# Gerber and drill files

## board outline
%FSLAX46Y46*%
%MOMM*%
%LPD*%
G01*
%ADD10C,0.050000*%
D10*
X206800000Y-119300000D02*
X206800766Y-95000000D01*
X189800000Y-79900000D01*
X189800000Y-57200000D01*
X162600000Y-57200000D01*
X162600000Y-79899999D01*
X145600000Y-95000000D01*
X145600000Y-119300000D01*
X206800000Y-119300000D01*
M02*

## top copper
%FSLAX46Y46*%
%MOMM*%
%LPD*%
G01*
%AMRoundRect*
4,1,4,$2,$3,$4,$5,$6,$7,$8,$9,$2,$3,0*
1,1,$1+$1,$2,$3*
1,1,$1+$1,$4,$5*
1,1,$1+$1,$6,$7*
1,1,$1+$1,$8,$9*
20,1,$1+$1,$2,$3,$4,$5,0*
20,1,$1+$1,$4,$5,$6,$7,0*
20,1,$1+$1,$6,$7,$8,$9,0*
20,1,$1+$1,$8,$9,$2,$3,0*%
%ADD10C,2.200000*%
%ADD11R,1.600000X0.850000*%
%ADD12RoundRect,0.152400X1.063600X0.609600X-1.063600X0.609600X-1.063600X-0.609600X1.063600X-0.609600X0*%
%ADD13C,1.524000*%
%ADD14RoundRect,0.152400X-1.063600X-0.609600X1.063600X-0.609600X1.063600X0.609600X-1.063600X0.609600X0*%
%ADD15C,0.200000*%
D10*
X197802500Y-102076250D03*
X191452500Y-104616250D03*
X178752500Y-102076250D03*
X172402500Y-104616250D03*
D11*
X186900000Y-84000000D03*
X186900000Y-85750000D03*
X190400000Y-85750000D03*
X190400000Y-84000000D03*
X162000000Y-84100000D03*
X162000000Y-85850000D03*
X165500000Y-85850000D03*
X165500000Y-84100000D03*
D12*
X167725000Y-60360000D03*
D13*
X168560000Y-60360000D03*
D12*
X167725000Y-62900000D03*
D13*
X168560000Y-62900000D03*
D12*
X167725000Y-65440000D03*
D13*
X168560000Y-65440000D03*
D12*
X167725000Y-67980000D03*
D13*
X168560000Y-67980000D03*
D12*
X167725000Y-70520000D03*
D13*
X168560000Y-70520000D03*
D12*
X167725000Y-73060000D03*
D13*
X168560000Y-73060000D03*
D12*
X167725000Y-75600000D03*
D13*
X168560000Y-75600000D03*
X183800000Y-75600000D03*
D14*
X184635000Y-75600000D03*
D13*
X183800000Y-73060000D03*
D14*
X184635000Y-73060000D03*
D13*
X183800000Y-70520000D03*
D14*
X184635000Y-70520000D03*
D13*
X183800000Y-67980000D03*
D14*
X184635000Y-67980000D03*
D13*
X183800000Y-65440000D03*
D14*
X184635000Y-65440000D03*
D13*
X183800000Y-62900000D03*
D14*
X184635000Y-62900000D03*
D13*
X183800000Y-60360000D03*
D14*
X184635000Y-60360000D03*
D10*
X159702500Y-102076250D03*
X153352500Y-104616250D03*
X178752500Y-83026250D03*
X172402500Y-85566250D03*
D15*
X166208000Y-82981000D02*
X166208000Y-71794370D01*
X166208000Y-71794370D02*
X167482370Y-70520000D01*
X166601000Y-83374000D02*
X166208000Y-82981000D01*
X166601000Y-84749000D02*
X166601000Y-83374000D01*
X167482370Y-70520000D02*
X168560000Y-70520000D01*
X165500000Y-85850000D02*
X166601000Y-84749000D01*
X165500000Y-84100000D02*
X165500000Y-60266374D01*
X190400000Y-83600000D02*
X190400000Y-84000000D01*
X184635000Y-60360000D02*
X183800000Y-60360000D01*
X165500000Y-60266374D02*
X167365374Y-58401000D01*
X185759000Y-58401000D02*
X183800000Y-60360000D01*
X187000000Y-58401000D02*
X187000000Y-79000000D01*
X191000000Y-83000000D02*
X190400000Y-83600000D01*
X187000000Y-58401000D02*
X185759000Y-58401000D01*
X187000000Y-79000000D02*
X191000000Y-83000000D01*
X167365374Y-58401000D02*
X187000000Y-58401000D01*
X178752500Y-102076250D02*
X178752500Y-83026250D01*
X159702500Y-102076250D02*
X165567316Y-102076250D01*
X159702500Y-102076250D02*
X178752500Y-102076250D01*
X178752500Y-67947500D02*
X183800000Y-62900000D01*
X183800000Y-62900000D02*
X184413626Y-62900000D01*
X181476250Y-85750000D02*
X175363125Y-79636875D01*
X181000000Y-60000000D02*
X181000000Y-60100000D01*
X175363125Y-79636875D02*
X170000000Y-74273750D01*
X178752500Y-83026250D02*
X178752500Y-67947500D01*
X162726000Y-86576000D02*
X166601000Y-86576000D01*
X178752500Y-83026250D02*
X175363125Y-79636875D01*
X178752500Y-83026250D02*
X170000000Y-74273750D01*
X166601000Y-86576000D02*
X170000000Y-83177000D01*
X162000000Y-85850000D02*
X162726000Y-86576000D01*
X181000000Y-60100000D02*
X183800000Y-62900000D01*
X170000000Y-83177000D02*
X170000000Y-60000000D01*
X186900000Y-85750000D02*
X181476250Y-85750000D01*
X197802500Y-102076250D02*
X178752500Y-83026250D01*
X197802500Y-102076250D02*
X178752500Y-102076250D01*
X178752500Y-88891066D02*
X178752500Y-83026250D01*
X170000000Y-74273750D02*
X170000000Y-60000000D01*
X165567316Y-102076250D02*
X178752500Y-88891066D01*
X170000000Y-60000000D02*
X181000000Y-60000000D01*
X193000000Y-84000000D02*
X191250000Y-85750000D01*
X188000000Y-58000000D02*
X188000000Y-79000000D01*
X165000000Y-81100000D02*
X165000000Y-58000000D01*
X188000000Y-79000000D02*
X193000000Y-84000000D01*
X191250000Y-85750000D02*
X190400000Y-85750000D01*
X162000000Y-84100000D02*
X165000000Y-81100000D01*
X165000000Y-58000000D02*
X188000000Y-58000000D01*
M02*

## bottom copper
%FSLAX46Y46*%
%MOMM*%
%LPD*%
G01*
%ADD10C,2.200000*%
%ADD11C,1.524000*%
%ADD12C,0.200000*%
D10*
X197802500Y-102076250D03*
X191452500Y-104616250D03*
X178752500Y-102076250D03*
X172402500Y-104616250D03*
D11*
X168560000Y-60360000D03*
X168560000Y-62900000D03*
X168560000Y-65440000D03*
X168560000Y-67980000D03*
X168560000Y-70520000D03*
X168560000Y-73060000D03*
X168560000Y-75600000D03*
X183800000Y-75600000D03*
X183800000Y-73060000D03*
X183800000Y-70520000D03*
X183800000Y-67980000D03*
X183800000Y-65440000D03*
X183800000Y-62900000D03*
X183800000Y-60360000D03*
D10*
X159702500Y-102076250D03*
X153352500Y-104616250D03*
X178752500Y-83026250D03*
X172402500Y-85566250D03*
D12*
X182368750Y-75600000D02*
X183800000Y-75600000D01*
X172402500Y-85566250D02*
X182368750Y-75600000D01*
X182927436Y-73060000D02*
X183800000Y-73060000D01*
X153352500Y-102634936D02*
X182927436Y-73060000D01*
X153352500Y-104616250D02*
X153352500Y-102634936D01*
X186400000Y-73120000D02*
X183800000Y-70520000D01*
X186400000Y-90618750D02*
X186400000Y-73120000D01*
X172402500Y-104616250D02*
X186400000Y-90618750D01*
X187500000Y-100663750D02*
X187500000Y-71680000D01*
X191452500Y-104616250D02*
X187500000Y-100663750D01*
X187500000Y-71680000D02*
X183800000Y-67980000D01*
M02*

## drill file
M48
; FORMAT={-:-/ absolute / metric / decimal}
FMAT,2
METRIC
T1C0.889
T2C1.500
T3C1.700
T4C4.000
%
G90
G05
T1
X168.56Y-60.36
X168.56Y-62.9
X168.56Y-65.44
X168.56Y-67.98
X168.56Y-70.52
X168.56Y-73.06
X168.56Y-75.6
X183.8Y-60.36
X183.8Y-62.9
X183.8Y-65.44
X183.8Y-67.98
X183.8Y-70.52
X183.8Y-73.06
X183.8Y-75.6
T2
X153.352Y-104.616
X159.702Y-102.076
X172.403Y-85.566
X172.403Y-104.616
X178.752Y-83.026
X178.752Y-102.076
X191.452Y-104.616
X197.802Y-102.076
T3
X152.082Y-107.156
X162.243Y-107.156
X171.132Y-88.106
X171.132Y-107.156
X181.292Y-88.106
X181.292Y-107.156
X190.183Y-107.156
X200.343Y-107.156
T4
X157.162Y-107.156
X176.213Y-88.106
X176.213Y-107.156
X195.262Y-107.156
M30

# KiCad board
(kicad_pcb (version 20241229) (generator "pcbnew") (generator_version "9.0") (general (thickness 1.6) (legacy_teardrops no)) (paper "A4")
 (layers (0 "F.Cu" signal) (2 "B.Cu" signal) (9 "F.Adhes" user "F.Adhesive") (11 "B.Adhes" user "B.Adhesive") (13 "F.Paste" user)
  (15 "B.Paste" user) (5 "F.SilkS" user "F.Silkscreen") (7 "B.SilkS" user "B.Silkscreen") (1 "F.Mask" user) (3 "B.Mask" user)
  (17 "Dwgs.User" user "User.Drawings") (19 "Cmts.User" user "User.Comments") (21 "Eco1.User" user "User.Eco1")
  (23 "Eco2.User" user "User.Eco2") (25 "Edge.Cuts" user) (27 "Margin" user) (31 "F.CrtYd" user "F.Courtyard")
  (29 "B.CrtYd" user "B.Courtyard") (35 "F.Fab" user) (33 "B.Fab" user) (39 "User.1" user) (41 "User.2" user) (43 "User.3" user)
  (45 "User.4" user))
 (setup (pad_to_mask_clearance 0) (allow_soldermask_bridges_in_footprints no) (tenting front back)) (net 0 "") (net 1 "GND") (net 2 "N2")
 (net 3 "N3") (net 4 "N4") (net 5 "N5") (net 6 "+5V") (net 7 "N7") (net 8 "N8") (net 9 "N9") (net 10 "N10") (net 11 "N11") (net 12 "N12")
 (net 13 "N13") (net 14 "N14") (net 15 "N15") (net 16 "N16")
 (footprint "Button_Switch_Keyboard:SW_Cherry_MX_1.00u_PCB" (layer "F.Cu") (at 197.8025 102.07625)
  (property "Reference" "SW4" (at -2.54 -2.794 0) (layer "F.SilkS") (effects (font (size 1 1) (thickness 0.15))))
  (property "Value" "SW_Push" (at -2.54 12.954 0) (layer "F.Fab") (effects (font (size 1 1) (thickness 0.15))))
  (pad "" np_thru_hole circle (at -7.62 5.08) (size 1.7 1.7) (drill 1.7) (layers "*.Cu" "*.Mask"))
  (pad "" np_thru_hole circle (at -2.54 5.08) (size 4 4) (drill 4) (layers "*.Cu" "*.Mask"))
  (pad "" np_thru_hole circle (at 2.54 5.08) (size 1.7 1.7) (drill 1.7) (layers "*.Cu" "*.Mask"))
  (pad "1" thru_hole circle (at 0 0) (size 2.2 2.2) (drill 1.5) (layers "*.Cu" "*.Mask") (remove_unused_layers no) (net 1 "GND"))
  (pad "2" thru_hole circle (at -6.35 2.54) (size 2.2 2.2) (drill 1.5) (layers "*.Cu" "*.Mask") (remove_unused_layers no) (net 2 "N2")))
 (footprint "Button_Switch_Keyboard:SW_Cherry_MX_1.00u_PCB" (layer "F.Cu") (at 178.7525 102.07625)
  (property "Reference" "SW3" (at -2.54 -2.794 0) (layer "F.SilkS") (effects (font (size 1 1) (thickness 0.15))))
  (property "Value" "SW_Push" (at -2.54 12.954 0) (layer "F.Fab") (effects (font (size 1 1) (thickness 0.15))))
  (pad "" np_thru_hole circle (at -7.62 5.08) (size 1.7 1.7) (drill 1.7) (layers "*.Cu" "*.Mask"))
  (pad "" np_thru_hole circle (at -2.54 5.08) (size 4 4) (drill 4) (layers "*.Cu" "*.Mask"))
  (pad "" np_thru_hole circle (at 2.54 5.08) (size 1.7 1.7) (drill 1.7) (layers "*.Cu" "*.Mask"))
  (pad "1" thru_hole circle (at 0 0) (size 2.2 2.2) (drill 1.5) (layers "*.Cu" "*.Mask") (remove_unused_layers no) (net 1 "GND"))
  (pad "2" thru_hole circle (at -6.35 2.54) (size 2.2 2.2) (drill 1.5) (layers "*.Cu" "*.Mask") (remove_unused_layers no) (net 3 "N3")))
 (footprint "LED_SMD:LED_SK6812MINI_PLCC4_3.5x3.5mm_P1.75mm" (layer "F.Cu") (at 188.65 84.875)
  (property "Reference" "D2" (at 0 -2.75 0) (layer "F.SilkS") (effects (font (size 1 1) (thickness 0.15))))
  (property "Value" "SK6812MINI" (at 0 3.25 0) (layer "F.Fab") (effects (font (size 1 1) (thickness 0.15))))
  (pad "1" smd rect (at -1.75 -0.875) (size 1.6 0.85) (layers "F.Cu" "F.Mask" "F.Paste") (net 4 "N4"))
  (pad "2" smd rect (at -1.75 0.875) (size 1.6 0.85) (layers "F.Cu" "F.Mask" "F.Paste") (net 1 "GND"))
  (pad "3" smd rect (at 1.75 0.875) (size 1.6 0.85) (layers "F.Cu" "F.Mask" "F.Paste") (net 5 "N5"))
  (pad "4" smd rect (at 1.75 -0.875) (size 1.6 0.85) (layers "F.Cu" "F.Mask" "F.Paste") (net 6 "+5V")))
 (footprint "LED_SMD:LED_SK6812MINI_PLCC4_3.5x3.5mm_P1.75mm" (layer "F.Cu") (at 163.75 84.975)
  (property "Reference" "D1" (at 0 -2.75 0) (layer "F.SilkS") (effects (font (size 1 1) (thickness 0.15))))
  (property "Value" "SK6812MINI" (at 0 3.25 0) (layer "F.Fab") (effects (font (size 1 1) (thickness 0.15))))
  (pad "1" smd rect (at -1.75 -0.875) (size 1.6 0.85) (layers "F.Cu" "F.Mask" "F.Paste") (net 5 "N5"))
  (pad "2" smd rect (at -1.75 0.875) (size 1.6 0.85) (layers "F.Cu" "F.Mask" "F.Paste") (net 1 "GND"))
  (pad "3" smd rect (at 1.75 0.875) (size 1.6 0.85) (layers "F.Cu" "F.Mask" "F.Paste") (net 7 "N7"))
  (pad "4" smd rect (at 1.75 -0.875) (size 1.6 0.85) (layers "F.Cu" "F.Mask" "F.Paste") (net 6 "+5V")))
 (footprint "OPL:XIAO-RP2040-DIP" (layer "F.Cu") (at 176.18 67.98)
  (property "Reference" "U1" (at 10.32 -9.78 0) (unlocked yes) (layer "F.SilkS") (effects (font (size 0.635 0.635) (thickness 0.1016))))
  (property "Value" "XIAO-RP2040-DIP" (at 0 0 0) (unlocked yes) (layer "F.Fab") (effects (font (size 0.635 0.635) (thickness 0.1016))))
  (pad "1" smd roundrect (at -8.455 -7.62 180) (size 2.432 1.524) (layers "F.Cu" "F.Mask") (roundrect_rratio 0.1) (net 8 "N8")
   (thermal_bridge_angle 45))
  (pad "1" thru_hole circle (at -7.62 -7.62 180) (size 1.524 1.524) (drill 0.889) (layers "*.Cu" "*.Mask") (remove_unused_layers no)
   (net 8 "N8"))
  (pad "2" smd roundrect (at -8.455 -5.08 180) (size 2.432 1.524) (layers "F.Cu" "F.Mask") (roundrect_rratio 0.1) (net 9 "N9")
   (thermal_bridge_angle 45))
  (pad "2" thru_hole circle (at -7.62 -5.08 180) (size 1.524 1.524) (drill 0.889) (layers "*.Cu" "*.Mask") (remove_unused_layers no)
   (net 9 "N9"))
  (pad "3" smd roundrect (at -8.455 -2.54 180) (size 2.432 1.524) (layers "F.Cu" "F.Mask") (roundrect_rratio 0.1) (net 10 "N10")
   (thermal_bridge_angle 45))
  (pad "3" thru_hole circle (at -7.62 -2.54 180) (size 1.524 1.524) (drill 0.889) (layers "*.Cu" "*.Mask") (remove_unused_layers no)
   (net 10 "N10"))
  (pad "4" smd roundrect (at -8.455 0 180) (size 2.432 1.524) (layers "F.Cu" "F.Mask") (roundrect_rratio 0.1) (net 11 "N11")
   (thermal_bridge_angle 45))
  (pad "4" thru_hole circle (at -7.62 0 180) (size 1.524 1.524) (drill 0.889) (layers "*.Cu" "*.Mask") (remove_unused_layers no)
   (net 11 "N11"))
  (pad "5" smd roundrect (at -8.455 2.54 180) (size 2.432 1.524) (layers "F.Cu" "F.Mask") (roundrect_rratio 0.1) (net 7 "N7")
   (thermal_bridge_angle 45))
  (pad "5" thru_hole circle (at -7.62 2.54 180) (size 1.524 1.524) (drill 0.889) (layers "*.Cu" "*.Mask") (remove_unused_layers no)
   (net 7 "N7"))
  (pad "6" smd roundrect (at -8.455 5.08 180) (size 2.432 1.524) (layers "F.Cu" "F.Mask") (roundrect_rratio 0.1) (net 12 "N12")
   (thermal_bridge_angle 45))
  (pad "6" thru_hole circle (at -7.62 5.08 180) (size 1.524 1.524) (drill 0.889) (layers "*.Cu" "*.Mask") (remove_unused_layers no)
   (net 12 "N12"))
  (pad "7" smd roundrect (at -8.455 7.62 180) (size 2.432 1.524) (layers "F.Cu" "F.Mask") (roundrect_rratio 0.1) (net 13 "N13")
   (thermal_bridge_angle 45))
  (pad "7" thru_hole circle (at -7.62 7.62 180) (size 1.524 1.524) (drill 0.889) (layers "*.Cu" "*.Mask") (remove_unused_layers no)
   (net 13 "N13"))
  (pad "8" thru_hole circle (at 7.62 7.62) (size 1.524 1.524) (drill 0.889) (layers "*.Cu" "*.Mask") (remove_unused_layers no)
   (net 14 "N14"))
  (pad "8" smd roundrect (at 8.455 7.62) (size 2.432 1.524) (layers "F.Cu" "F.Mask") (roundrect_rratio 0.1) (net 14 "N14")
   (thermal_bridge_angle 45))
  (pad "9" thru_hole circle (at 7.62 5.08) (size 1.524 1.524) (drill 0.889) (layers "*.Cu" "*.Mask") (remove_unused_layers no)
   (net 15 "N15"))
  (pad "9" smd roundrect (at 8.455 5.08) (size 2.432 1.524) (layers "F.Cu" "F.Mask") (roundrect_rratio 0.1) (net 15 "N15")
   (thermal_bridge_angle 45))
  (pad "10" thru_hole circle (at 7.62 2.54) (size 1.524 1.524) (drill 0.889) (layers "*.Cu" "*.Mask") (remove_unused_layers no) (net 3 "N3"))
  (pad "10" smd roundrect (at 8.455 2.54) (size 2.432 1.524) (layers "F.Cu" "F.Mask") (roundrect_rratio 0.1) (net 3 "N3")
   (thermal_bridge_angle 45))
  (pad "11" thru_hole circle (at 7.62 0) (size 1.524 1.524) (drill 0.889) (layers "*.Cu" "*.Mask") (remove_unused_layers no) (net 2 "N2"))
  (pad "11" smd roundrect (at 8.455 0) (size 2.432 1.524) (layers "F.Cu" "F.Mask") (roundrect_rratio 0.1) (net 2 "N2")
   (thermal_bridge_angle 45))
  (pad "12" thru_hole circle (at 7.62 -2.54) (size 1.524 1.524) (drill 0.889) (layers "*.Cu" "*.Mask") (remove_unused_layers no)
   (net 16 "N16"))
  (pad "12" smd roundrect (at 8.455 -2.54) (size 2.432 1.524) (layers "F.Cu" "F.Mask") (roundrect_rratio 0.1) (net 16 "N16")
   (thermal_bridge_angle 45))
  (pad "13" thru_hole circle (at 7.62 -5.08) (size 1.524 1.524) (drill 0.889) (layers "*.Cu" "*.Mask") (remove_unused_layers no)
   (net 1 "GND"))
  (pad "13" smd roundrect (at 8.455 -5.08) (size 2.432 1.524) (layers "F.Cu" "F.Mask") (roundrect_rratio 0.1) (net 1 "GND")
   (thermal_bridge_angle 45))
  (pad "14" thru_hole circle (at 7.62 -7.62) (size 1.524 1.524) (drill 0.889) (layers "*.Cu" "*.Mask") (remove_unused_layers no)
   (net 6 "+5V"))
  (pad "14" smd roundrect (at 8.455 -7.62) (size 2.432 1.524) (layers "F.Cu" "F.Mask") (roundrect_rratio 0.1) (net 6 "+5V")
   (thermal_bridge_angle 45)))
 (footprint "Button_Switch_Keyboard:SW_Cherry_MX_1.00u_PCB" (layer "F.Cu") (at 159.7025 102.07625)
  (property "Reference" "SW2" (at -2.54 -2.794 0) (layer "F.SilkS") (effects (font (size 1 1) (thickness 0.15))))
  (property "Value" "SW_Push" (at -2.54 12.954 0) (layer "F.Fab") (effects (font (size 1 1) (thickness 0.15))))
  (pad "" np_thru_hole circle (at -7.62 5.08) (size 1.7 1.7) (drill 1.7) (layers "*.Cu" "*.Mask"))
  (pad "" np_thru_hole circle (at -2.54 5.08) (size 4 4) (drill 4) (layers "*.Cu" "*.Mask"))
  (pad "" np_thru_hole circle (at 2.54 5.08) (size 1.7 1.7) (drill 1.7) (layers "*.Cu" "*.Mask"))
  (pad "1" thru_hole circle (at 0 0) (size 2.2 2.2) (drill 1.5) (layers "*.Cu" "*.Mask") (remove_unused_layers no) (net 1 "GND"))
  (pad "2" thru_hole circle (at -6.35 2.54) (size 2.2 2.2) (drill 1.5) (layers "*.Cu" "*.Mask") (remove_unused_layers no) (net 15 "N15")))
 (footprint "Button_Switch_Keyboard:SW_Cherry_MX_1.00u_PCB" (layer "F.Cu") (at 178.7525 83.02625)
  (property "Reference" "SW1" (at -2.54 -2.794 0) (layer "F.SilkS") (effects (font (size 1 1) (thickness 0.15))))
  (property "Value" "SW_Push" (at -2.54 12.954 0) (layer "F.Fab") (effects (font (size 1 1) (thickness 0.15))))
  (pad "" np_thru_hole circle (at -7.62 5.08) (size 1.7 1.7) (drill 1.7) (layers "*.Cu" "*.Mask"))
  (pad "" np_thru_hole circle (at -2.54 5.08) (size 4 4) (drill 4) (layers "*.Cu" "*.Mask"))
  (pad "" np_thru_hole circle (at 2.54 5.08) (size 1.7 1.7) (drill 1.7) (layers "*.Cu" "*.Mask"))
  (pad "1" thru_hole circle (at 0 0) (size 2.2 2.2) (drill 1.5) (layers "*.Cu" "*.Mask") (remove_unused_layers no) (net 1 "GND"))
  (pad "2" thru_hole circle (at -6.35 2.54) (size 2.2 2.2) (drill 1.5) (layers "*.Cu" "*.Mask") (remove_unused_layers no) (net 14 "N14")))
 (gr_poly
  (pts (xy 206.8 119.3) (xy 206.800766 95) (xy 189.8 79.9) (xy 189.8 57.2) (xy 162.6 57.2) (xy 162.6 79.899999) (xy 145.6 95)
   (xy 145.6 119.3))
  (stroke (width 0.05) (type solid)) (fill no) (layer "Edge.Cuts"))
 (segment (start 166.208 82.981) (end 166.208 71.79437) (width 0.2) (layer "F.Cu") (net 7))
 (segment (start 166.208 71.79437) (end 167.48237 70.52) (width 0.2) (layer "F.Cu") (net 7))
 (segment (start 166.601 83.374) (end 166.208 82.981) (width 0.2) (layer "F.Cu") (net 7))
 (segment (start 166.601 84.749) (end 166.601 83.374) (width 0.2) (layer "F.Cu") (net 7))
 (segment (start 167.48237 70.52) (end 168.56 70.52) (width 0.2) (layer "F.Cu") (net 7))
 (segment (start 165.5 85.85) (end 166.601 84.749) (width 0.2) (layer "F.Cu") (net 7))
 (segment (start 165.5 84.1) (end 165.5 60.266374) (width 0.2) (layer "F.Cu") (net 6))
 (segment (start 190.4 83.6) (end 190.4 84) (width 0.2) (layer "F.Cu") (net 6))
 (segment (start 184.635 60.36) (end 183.8 60.36) (width 0.2) (layer "F.Cu") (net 6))
 (segment (start 165.5 60.266374) (end 167.365374 58.401) (width 0.2) (layer "F.Cu") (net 6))
 (segment (start 185.759 58.401) (end 183.8 60.36) (width 0.2) (layer "F.Cu") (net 6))
 (segment (start 187 58.401) (end 187 79) (width 0.2) (layer "F.Cu") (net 6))
 (segment (start 191 83) (end 190.4 83.6) (width 0.2) (layer "F.Cu") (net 6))
 (segment (start 187 58.401) (end 185.759 58.401) (width 0.2) (layer "F.Cu") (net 6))
 (segment (start 187 79) (end 191 83) (width 0.2) (layer "F.Cu") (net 6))
 (segment (start 167.365374 58.401) (end 187 58.401) (width 0.2) (layer "F.Cu") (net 6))
 (segment (start 178.7525 102.07625) (end 178.7525 83.02625) (width 0.2) (layer "F.Cu") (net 1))
 (segment (start 159.7025 102.07625) (end 165.567316 102.07625) (width 0.2) (layer "F.Cu") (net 1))
 (segment (start 159.7025 102.07625) (end 178.7525 102.07625) (width 0.2) (layer "F.Cu") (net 1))
 (segment (start 178.7525 67.9475) (end 183.8 62.9) (width 0.2) (layer "F.Cu") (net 1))
 (segment (start 183.8 62.9) (end 184.413626 62.9) (width 0.2) (layer "F.Cu") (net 1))
 (segment (start 181.47625 85.75) (end 175.363125 79.636875) (width 0.2) (layer "F.Cu") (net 1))
 (segment (start 181 60) (end 181 60.1) (width 0.2) (layer "F.Cu") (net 1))
 (segment (start 175.363125 79.636875) (end 170 74.27375) (width 0.2) (layer "F.Cu") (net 1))
 (segment (start 178.7525 83.02625) (end 178.7525 67.9475) (width 0.2) (layer "F.Cu") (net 1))
 (segment (start 162.726 86.576) (end 166.601 86.576) (width 0.2) (layer "F.Cu") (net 1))
 (segment (start 178.7525 83.02625) (end 175.363125 79.636875) (width 0.2) (layer "F.Cu") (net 1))
 (segment (start 178.7525 83.02625) (end 170 74.27375) (width 0.2) (layer "F.Cu") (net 1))
 (segment (start 166.601 86.576) (end 170 83.177) (width 0.2) (layer "F.Cu") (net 1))
 (segment (start 162 85.85) (end 162.726 86.576) (width 0.2) (layer "F.Cu") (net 1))
 (segment (start 181 60.1) (end 183.8 62.9) (width 0.2) (layer "F.Cu") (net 1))
 (segment (start 170 83.177) (end 170 60) (width 0.2) (layer "F.Cu") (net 1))
 (segment (start 186.9 85.75) (end 181.47625 85.75) (width 0.2) (layer "F.Cu") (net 1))
 (segment (start 197.8025 102.07625) (end 178.7525 83.02625) (width 0.2) (layer "F.Cu") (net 1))
 (segment (start 197.8025 102.07625) (end 178.7525 102.07625) (width 0.2) (layer "F.Cu") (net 1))
 (segment (start 178.7525 88.891066) (end 178.7525 83.02625) (width 0.2) (layer "F.Cu") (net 1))
 (segment (start 170 74.27375) (end 170 60) (width 0.2) (layer "F.Cu") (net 1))
 (segment (start 165.567316 102.07625) (end 178.7525 88.891066) (width 0.2) (layer "F.Cu") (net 1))
 (segment (start 170 60) (end 181 60) (width 0.2) (layer "F.Cu") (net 1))
 (segment (start 193 84) (end 191.25 85.75) (width 0.2) (layer "F.Cu") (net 5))
 (segment (start 188 58) (end 188 79) (width 0.2) (layer "F.Cu") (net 5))
 (segment (start 165 81.1) (end 165 58) (width 0.2) (layer "F.Cu") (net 5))
 (segment (start 188 79) (end 193 84) (width 0.2) (layer "F.Cu") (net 5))
 (segment (start 191.25 85.75) (end 190.4 85.75) (width 0.2) (layer "F.Cu") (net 5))
 (segment (start 162 84.1) (end 165 81.1) (width 0.2) (layer "F.Cu") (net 5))
 (segment (start 165 58) (end 188 58) (width 0.2) (layer "F.Cu") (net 5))
 (segment (start 182.36875 75.6) (end 183.8 75.6) (width 0.2) (layer "B.Cu") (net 14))
 (segment (start 172.4025 85.56625) (end 182.36875 75.6) (width 0.2) (layer "B.Cu") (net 14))
 (segment (start 182.927436 73.06) (end 183.8 73.06) (width 0.2) (layer "B.Cu") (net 15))
 (segment (start 153.3525 102.634936) (end 182.927436 73.06) (width 0.2) (layer "B.Cu") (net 15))
 (segment (start 153.3525 104.61625) (end 153.3525 102.634936) (width 0.2) (layer "B.Cu") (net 15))
 (segment (start 186.4 73.12) (end 183.8 70.52) (width 0.2) (layer "B.Cu") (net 3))
 (segment (start 186.4 90.61875) (end 186.4 73.12) (width 0.2) (layer "B.Cu") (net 3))
 (segment (start 172.4025 104.61625) (end 186.4 90.61875) (width 0.2) (layer "B.Cu") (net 3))
 (segment (start 187.5 100.66375) (end 187.5 71.68) (width 0.2) (layer "B.Cu") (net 2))
 (segment (start 191.4525 104.61625) (end 187.5 100.66375) (width 0.2) (layer "B.Cu") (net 2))
 (segment (start 187.5 71.68) (end 183.8 67.98) (width 0.2) (layer "B.Cu") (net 2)))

